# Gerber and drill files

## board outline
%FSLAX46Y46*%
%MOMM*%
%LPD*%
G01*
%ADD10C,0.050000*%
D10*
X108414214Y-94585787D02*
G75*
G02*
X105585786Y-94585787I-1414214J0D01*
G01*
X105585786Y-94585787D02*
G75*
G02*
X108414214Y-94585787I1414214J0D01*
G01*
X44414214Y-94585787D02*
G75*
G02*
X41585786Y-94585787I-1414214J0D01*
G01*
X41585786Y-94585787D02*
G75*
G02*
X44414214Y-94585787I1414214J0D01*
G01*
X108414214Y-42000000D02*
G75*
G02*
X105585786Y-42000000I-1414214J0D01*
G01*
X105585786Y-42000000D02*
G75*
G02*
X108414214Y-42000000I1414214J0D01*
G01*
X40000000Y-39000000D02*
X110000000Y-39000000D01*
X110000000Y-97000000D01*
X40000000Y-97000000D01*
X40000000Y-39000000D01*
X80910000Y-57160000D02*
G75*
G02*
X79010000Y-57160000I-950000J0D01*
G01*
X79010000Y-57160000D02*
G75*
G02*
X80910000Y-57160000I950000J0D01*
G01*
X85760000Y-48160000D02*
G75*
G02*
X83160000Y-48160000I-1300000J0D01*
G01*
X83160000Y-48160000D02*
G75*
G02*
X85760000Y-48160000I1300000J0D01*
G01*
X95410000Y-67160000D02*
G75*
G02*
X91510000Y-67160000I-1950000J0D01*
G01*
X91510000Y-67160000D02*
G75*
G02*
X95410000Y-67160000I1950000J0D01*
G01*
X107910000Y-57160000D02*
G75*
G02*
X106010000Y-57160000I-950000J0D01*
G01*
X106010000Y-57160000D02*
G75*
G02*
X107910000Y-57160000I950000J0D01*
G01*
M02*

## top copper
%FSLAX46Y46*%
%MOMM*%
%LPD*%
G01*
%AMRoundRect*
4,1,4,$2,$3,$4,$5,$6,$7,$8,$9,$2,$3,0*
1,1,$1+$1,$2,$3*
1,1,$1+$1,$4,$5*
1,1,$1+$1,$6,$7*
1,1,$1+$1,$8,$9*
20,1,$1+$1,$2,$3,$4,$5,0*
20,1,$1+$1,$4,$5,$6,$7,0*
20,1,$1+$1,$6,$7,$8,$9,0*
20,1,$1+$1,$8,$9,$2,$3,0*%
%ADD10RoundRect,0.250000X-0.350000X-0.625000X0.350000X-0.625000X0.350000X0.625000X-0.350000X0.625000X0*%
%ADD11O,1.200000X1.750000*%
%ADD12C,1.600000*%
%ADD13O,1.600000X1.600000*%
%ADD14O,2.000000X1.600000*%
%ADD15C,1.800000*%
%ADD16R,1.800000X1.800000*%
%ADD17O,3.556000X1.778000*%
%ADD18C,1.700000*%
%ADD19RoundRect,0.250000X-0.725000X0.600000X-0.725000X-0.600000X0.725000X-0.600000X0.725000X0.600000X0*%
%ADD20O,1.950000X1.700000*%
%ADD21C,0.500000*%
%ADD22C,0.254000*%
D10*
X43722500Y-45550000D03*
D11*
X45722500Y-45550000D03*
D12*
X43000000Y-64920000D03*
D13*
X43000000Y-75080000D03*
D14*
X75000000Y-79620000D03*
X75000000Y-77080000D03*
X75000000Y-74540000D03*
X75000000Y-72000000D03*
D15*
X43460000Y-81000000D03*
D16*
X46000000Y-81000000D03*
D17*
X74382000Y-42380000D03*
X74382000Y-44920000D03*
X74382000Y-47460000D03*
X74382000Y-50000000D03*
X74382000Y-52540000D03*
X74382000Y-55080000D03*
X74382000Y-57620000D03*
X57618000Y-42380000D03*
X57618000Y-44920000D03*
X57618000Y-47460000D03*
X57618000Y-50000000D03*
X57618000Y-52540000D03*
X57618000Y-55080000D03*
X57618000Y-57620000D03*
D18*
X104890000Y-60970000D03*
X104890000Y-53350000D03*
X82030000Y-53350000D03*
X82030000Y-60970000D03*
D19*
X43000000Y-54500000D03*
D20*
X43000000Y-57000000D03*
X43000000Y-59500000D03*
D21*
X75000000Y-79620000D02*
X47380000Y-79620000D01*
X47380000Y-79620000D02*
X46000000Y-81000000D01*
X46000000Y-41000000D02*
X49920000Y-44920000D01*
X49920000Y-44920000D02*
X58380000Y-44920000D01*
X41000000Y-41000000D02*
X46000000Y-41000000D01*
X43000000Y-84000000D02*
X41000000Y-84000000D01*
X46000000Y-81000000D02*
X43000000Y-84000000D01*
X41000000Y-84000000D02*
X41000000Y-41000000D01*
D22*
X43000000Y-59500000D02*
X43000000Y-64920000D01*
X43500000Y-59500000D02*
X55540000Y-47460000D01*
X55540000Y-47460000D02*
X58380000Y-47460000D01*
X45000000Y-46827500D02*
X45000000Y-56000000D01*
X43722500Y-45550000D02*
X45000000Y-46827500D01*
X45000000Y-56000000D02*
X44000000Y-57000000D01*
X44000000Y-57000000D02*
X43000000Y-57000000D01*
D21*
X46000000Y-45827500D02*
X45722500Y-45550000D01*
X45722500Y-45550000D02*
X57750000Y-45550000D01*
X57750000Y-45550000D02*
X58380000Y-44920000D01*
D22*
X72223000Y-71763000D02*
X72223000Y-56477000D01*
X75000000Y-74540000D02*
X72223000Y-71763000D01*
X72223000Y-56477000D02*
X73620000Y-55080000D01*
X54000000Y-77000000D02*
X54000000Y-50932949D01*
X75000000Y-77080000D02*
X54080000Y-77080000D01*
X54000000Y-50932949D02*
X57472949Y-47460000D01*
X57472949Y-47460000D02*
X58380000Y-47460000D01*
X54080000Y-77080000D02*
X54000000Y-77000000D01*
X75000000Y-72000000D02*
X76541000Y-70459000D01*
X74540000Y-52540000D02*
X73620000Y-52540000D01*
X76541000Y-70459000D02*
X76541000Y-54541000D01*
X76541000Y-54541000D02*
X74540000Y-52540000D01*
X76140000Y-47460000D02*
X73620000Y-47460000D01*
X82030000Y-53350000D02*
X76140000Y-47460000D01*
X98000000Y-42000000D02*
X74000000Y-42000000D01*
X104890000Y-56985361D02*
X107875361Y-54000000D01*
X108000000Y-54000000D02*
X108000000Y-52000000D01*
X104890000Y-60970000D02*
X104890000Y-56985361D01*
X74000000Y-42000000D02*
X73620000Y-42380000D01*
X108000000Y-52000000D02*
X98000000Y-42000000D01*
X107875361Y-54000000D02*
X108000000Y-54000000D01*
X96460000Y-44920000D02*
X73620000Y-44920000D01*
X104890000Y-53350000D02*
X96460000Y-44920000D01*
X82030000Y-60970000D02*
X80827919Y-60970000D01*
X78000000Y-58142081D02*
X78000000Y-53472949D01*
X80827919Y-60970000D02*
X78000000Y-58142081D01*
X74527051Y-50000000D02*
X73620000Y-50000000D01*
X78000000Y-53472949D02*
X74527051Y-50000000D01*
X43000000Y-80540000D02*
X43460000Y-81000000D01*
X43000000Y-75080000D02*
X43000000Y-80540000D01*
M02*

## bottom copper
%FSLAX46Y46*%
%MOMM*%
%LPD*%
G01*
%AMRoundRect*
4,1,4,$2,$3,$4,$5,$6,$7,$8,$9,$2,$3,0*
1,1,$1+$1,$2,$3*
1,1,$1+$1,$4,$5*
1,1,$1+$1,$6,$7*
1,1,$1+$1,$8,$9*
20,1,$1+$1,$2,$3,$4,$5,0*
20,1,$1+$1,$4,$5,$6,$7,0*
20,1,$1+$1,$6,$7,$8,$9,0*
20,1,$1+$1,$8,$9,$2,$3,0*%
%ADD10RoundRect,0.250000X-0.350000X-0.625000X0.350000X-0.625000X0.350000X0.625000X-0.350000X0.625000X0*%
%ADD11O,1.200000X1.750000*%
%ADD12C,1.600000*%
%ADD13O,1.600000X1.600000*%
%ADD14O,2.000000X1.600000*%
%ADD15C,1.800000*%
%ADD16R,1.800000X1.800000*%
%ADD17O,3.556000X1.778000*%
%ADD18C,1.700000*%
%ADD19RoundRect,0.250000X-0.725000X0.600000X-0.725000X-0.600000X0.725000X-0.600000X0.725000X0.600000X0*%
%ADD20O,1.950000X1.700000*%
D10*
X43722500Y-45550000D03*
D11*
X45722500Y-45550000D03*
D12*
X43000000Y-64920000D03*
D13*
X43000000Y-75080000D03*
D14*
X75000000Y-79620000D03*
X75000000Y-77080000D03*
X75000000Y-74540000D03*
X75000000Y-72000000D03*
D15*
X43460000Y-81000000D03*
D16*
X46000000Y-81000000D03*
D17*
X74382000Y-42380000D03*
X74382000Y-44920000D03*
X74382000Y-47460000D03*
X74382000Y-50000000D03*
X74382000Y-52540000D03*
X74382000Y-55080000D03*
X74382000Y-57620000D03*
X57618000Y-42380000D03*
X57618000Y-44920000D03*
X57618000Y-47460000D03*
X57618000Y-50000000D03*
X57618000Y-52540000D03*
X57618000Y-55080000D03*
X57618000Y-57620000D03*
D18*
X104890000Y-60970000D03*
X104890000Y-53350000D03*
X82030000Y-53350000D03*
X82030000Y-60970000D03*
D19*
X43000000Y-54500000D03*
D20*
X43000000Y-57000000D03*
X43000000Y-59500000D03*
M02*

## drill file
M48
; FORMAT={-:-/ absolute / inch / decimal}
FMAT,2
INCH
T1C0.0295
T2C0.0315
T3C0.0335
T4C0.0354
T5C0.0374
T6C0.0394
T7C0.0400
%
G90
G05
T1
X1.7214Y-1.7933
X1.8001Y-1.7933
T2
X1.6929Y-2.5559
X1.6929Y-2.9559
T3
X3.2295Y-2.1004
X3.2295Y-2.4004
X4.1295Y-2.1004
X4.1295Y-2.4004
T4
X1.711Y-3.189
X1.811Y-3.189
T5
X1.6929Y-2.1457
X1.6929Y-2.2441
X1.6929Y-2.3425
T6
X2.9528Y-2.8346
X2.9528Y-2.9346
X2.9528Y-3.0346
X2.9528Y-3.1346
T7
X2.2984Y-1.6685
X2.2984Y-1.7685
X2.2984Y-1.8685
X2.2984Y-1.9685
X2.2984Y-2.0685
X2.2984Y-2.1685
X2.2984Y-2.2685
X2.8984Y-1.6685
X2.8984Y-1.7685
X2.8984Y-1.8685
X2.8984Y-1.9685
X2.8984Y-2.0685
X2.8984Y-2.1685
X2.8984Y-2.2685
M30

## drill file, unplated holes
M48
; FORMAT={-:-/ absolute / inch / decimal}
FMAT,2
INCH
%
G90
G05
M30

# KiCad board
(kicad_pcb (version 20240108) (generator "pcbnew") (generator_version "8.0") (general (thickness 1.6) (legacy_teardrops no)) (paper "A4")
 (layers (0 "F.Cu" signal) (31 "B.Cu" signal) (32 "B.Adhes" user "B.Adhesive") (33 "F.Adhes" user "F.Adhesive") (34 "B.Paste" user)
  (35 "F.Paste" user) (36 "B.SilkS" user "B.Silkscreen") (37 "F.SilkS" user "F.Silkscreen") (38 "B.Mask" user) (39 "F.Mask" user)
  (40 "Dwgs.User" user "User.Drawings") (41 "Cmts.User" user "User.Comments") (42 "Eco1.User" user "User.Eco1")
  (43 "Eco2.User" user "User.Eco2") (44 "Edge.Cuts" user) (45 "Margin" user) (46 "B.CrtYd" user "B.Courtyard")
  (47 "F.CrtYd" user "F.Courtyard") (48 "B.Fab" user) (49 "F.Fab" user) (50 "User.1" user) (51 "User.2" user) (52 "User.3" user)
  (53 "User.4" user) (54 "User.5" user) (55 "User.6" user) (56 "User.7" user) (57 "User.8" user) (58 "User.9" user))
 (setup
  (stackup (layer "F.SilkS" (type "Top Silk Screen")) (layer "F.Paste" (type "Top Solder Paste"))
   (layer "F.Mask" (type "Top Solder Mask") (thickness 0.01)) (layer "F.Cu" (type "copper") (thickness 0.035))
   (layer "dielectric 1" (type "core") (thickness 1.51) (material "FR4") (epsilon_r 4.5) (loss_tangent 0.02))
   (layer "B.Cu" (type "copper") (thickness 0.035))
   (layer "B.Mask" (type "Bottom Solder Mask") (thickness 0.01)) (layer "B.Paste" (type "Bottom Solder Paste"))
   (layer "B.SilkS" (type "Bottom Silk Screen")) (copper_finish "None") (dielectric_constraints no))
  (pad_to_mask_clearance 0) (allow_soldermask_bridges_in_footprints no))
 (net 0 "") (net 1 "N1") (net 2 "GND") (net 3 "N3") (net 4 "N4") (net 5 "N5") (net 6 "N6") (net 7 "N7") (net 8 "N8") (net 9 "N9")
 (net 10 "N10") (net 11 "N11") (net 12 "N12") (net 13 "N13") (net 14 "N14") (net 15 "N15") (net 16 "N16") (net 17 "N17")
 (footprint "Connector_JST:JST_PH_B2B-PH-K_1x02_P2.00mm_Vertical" (layer "B.Cu") (at 43.7225 45.55)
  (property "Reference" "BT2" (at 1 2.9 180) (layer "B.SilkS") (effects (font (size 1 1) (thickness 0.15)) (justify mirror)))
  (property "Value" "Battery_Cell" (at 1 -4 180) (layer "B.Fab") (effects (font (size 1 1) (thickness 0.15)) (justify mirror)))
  (pad "1" thru_hole roundrect (at 0 0) (size 1.2 1.75) (drill 0.75) (layers "*.Cu" "*.Mask") (remove_unused_layers no)
   (roundrect_rratio 0.208333) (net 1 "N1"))
  (pad "2" thru_hole oval (at 2 0) (size 1.2 1.75) (drill 0.75) (layers "*.Cu" "*.Mask") (remove_unused_layers no) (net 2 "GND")))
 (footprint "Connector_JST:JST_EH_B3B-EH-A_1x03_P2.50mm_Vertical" (layer "B.Cu") (at 43 54.5 -90)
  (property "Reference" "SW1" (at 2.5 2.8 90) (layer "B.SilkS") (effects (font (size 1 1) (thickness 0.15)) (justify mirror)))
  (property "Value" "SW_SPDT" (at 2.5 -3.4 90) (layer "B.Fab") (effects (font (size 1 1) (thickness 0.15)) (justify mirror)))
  (pad "1" thru_hole roundrect (at 0 0 270) (size 1.7 1.95) (drill 0.95) (layers "*.Cu" "*.Mask") (remove_unused_layers no)
   (roundrect_rratio 0.147059) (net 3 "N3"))
  (pad "2" thru_hole oval (at 2.5 0 270) (size 1.7 1.95) (drill 0.95) (layers "*.Cu" "*.Mask") (remove_unused_layers no) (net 1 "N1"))
  (pad "3" thru_hole oval (at 5 0 270) (size 1.7 1.95) (drill 0.95) (layers "*.Cu" "*.Mask") (remove_unused_layers no) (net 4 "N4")))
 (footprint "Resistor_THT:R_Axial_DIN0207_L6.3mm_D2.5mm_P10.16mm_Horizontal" (layer "B.Cu") (at 43 64.92 -90)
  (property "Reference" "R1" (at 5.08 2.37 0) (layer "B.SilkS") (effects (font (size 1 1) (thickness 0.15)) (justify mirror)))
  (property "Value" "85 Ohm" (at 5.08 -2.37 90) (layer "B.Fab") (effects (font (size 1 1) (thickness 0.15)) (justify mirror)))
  (pad "1" thru_hole circle (at 0 0 270) (size 1.6 1.6) (drill 0.8) (layers "*.Cu" "*.Mask") (remove_unused_layers no) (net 4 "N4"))
  (pad "2" thru_hole oval (at 10.16 0 270) (size 1.6 1.6) (drill 0.8) (layers "*.Cu" "*.Mask") (remove_unused_layers no) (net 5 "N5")))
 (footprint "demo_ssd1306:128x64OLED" (layer "B.Cu") (at 64.4 76 90)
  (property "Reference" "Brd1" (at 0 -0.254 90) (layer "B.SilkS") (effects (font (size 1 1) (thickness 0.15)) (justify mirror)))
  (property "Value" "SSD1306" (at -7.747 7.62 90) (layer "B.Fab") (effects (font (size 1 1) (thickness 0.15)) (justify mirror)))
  (pad "1" thru_hole oval (at -3.62 10.6) (size 2 1.6) (drill 1) (layers "*.Cu" "*.Mask") (remove_unused_layers no) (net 2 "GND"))
  (pad "2" thru_hole oval (at -1.08 10.6) (size 2 1.6) (drill 1) (layers "*.Cu" "*.Mask") (remove_unused_layers no) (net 4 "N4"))
  (pad "3" thru_hole oval (at 1.46 10.6) (size 2 1.6) (drill 1) (layers "*.Cu" "*.Mask") (remove_unused_layers no) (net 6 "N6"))
  (pad "4" thru_hole oval (at 4 10.6) (size 2 1.6) (drill 1) (layers "*.Cu" "*.Mask") (remove_unused_layers no) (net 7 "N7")))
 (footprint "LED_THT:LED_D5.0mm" (layer "B.Cu") (at 46 81 180)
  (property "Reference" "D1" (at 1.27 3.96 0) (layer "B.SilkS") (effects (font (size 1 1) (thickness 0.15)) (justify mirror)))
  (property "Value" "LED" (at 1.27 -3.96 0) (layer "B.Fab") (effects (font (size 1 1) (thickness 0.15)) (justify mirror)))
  (pad "1" thru_hole rect (at 0 0 180) (size 1.8 1.8) (drill 0.9) (layers "*.Cu" "*.Mask") (remove_unused_layers no) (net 2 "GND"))
  (pad "2" thru_hole circle (at 2.54 0 180) (size 1.8 1.8) (drill 0.9) (layers "*.Cu" "*.Mask") (remove_unused_layers no) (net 5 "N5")))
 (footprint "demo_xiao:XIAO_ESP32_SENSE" (layer "B.Cu") (at 66 50 180)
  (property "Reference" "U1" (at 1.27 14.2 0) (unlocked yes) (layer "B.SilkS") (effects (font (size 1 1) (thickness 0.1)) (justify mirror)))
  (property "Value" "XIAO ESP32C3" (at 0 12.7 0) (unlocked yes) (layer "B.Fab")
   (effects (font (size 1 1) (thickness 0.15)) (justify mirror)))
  (pad "1" thru_hole oval (at -7.62 7.62 180) (size 3.556 1.778) (drill 1.016 (offset -0.762 0)) (layers "*.Cu" "*.Mask")
   (remove_unused_layers no) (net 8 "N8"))
  (pad "2" thru_hole oval (at -7.62 5.08 180) (size 3.556 1.778) (drill 1.016 (offset -0.762 0)) (layers "*.Cu" "*.Mask")
   (remove_unused_layers no) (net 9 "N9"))
  (pad "3" thru_hole oval (at -7.62 2.54 180) (size 3.556 1.778) (drill 1.016 (offset -0.762 0)) (layers "*.Cu" "*.Mask")
   (remove_unused_layers no) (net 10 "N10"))
  (pad "4" thru_hole oval (at -7.62 0 180) (size 3.556 1.778) (drill 1.016 (offset -0.762 0)) (layers "*.Cu" "*.Mask")
   (remove_unused_layers no) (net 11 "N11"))
  (pad "5" thru_hole oval (at -7.62 -2.54 180) (size 3.556 1.778) (drill 1.016 (offset -0.762 0)) (layers "*.Cu" "*.Mask")
   (remove_unused_layers no) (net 7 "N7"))
  (pad "6" thru_hole oval (at -7.62 -5.08 180) (size 3.556 1.778) (drill 1.016 (offset -0.762 0)) (layers "*.Cu" "*.Mask")
   (remove_unused_layers no) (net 6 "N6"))
  (pad "7" thru_hole oval (at -7.62 -7.62 180) (size 3.556 1.778) (drill 1.016 (offset -0.762 0)) (layers "*.Cu" "*.Mask")
   (remove_unused_layers no) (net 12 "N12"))
  (pad "8" thru_hole oval (at 7.62 7.62 180) (size 3.556 1.778) (drill 1.016 (offset 0.762 0)) (layers "*.Cu" "*.Mask")
   (remove_unused_layers no) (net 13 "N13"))
  (pad "9" thru_hole oval (at 7.62 5.08 180) (size 3.556 1.778) (drill 1.016 (offset 0.762 0)) (layers "*.Cu" "*.Mask")
   (remove_unused_layers no) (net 2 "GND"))
  (pad "10" thru_hole oval (at 7.62 2.54 180) (size 3.556 1.778) (drill 1.016 (offset 0.762 0)) (layers "*.Cu" "*.Mask")
   (remove_unused_layers no) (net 4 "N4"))
  (pad "11" thru_hole oval (at 7.62 0 180) (size 3.556 1.778) (drill 1.016 (offset 0.762 0)) (layers "*.Cu" "*.Mask")
   (remove_unused_layers no) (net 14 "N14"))
  (pad "12" thru_hole oval (at 7.62 -2.54 180) (size 3.556 1.778) (drill 1.016 (offset 0.762 0)) (layers "*.Cu" "*.Mask")
   (remove_unused_layers no) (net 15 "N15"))
  (pad "13" thru_hole oval (at 7.62 -5.08 180) (size 3.556 1.778) (drill 1.016 (offset 0.762 0)) (layers "*.Cu" "*.Mask")
   (remove_unused_layers no) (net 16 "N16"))
  (pad "14" thru_hole oval (at 7.62 -7.62 180) (size 3.556 1.778) (drill 1.016 (offset 0.762 0)) (layers "*.Cu" "*.Mask")
   (remove_unused_layers no) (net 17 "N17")))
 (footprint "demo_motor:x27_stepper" (layer "B.Cu") (at 96 47)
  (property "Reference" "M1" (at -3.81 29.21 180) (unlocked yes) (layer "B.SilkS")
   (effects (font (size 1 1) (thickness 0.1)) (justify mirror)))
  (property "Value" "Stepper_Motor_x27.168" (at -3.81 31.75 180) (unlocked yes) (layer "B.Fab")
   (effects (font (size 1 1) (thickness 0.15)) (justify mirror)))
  (fp_circle (center -16.04 10.16) (end -15.09 10.16) (stroke (width 0.05) (type default)) (fill none) (layer "Edge.Cuts"))
  (fp_circle (center -11.54 1.16) (end -10.24 1.16) (stroke (width 0.05) (type default)) (fill none) (layer "Edge.Cuts"))
  (fp_circle (center -2.54 20.16) (end -0.59 20.16) (stroke (width 0.05) (type default)) (fill none) (layer "Edge.Cuts"))
  (fp_circle (center 10.96 10.16) (end 11.91 10.16) (stroke (width 0.05) (type default)) (fill none) (layer "Edge.Cuts"))
  (pad "1" thru_hole circle (at 8.89 13.97) (size 1.7 1.7) (drill 0.85) (layers "*.Cu" "*.Mask") (remove_unused_layers no) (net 8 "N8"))
  (pad "2" thru_hole circle (at 8.89 6.35) (size 1.7 1.7) (drill 0.85) (layers "*.Cu" "*.Mask") (remove_unused_layers no) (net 9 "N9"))
  (pad "3" thru_hole circle (at -13.97 6.35) (size 1.7 1.7) (drill 0.85) (layers "*.Cu" "*.Mask") (remove_unused_layers no) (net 10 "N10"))
  (pad "4" thru_hole circle (at -13.97 13.97) (size 1.7 1.7) (drill 0.85) (layers "*.Cu" "*.Mask") (remove_unused_layers no) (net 11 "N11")))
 (gr_rect (start 40 39) (end 110 97) (stroke (width 0.05) (type default)) (fill none) (layer "Edge.Cuts"))
 (gr_circle (center 43 94.585787) (end 44 95.585787) (stroke (width 0.05) (type default)) (fill none) (layer "Edge.Cuts"))
 (gr_circle (center 107 94.585787) (end 108 95.585787) (stroke (width 0.05) (type default)) (fill none) (layer "Edge.Cuts"))
 (gr_circle (center 107 42) (end 108 43) (stroke (width 0.05) (type default)) (fill none) (layer "Edge.Cuts"))
 (segment (start 72.223 71.763) (end 72.223 56.477) (width 0.254) (layer "F.Cu") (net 6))
 (segment (start 75 74.54) (end 72.223 71.763) (width 0.254) (layer "F.Cu") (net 6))
 (segment (start 72.223 56.477) (end 73.62 55.08) (width 0.254) (layer "F.Cu") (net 6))
 (segment (start 54 77) (end 54 50.932949) (width 0.254) (layer "F.Cu") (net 4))
 (segment (start 75 77.08) (end 54.08 77.08) (width 0.254) (layer "F.Cu") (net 4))
 (segment (start 43.5 59.5) (end 55.54 47.46) (width 0.254) (layer "F.Cu") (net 4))
 (segment (start 54 50.932949) (end 57.472949 47.46) (width 0.254) (layer "F.Cu") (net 4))
 (segment (start 57.472949 47.46) (end 58.38 47.46) (width 0.254) (layer "F.Cu") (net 4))
 (segment (start 54.08 77.08) (end 54 77) (width 0.254) (layer "F.Cu") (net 4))
 (segment (start 55.54 47.46) (end 58.38 47.46) (width 0.254) (layer "F.Cu") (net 4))
 (segment (start 43 59.5) (end 43 64.92) (width 0.254) (layer "F.Cu") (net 4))
 (segment (start 43 84) (end 41 84) (width 0.5) (layer "F.Cu") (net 2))
 (segment (start 46 41) (end 49.92 44.92) (width 0.5) (layer "F.Cu") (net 2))
 (segment (start 46 81) (end 43 84) (width 0.5) (layer "F.Cu") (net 2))
 (segment (start 75 79.62) (end 47.38 79.62) (width 0.5) (layer "F.Cu") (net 2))
 (segment (start 49.92 44.92) (end 58.38 44.92) (width 0.5) (layer "F.Cu") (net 2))
 (segment (start 46 45.8275) (end 45.7225 45.55) (width 0.5) (layer "F.Cu") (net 2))
 (segment (start 41 41) (end 46 41) (width 0.5) (layer "F.Cu") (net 2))
 (segment (start 47.38 79.62) (end 46 81) (width 0.5) (layer "F.Cu") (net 2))
 (segment (start 45.7225 45.55) (end 57.75 45.55) (width 0.5) (layer "F.Cu") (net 2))
 (segment (start 57.75 45.55) (end 58.38 44.92) (width 0.5) (layer "F.Cu") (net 2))
 (segment (start 41 84) (end 41 41) (width 0.5) (layer "F.Cu") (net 2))
 (segment (start 75 72) (end 76.541 70.459) (width 0.254) (layer "F.Cu") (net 7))
 (segment (start 74.54 52.54) (end 73.62 52.54) (width 0.254) (layer "F.Cu") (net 7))
 (segment (start 76.541 70.459) (end 76.541 54.541) (width 0.254) (layer "F.Cu") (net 7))
 (segment (start 76.541 54.541) (end 74.54 52.54) (width 0.254) (layer "F.Cu") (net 7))
 (segment (start 44 57) (end 43 57) (width 0.254) (layer "F.Cu") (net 1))
 (segment (start 45 46.8275) (end 45 56) (width 0.254) (layer "F.Cu") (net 1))
 (segment (start 43.7225 45.55) (end 45 46.8275) (width 0.254) (layer "F.Cu") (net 1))
 (segment (start 45 56) (end 44 57) (width 0.254) (layer "F.Cu") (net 1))
 (segment (start 43 75.08) (end 43 80.54) (width 0.254) (layer "F.Cu") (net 5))
 (segment (start 43 80.54) (end 43.46 81) (width 0.254) (layer "F.Cu") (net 5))
 (segment (start 76.14 47.46) (end 73.62 47.46) (width 0.254) (layer "F.Cu") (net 10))
 (segment (start 82.03 53.35) (end 76.14 47.46) (width 0.254) (layer "F.Cu") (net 10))
 (segment (start 98 42) (end 74 42) (width 0.254) (layer "F.Cu") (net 8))
 (segment (start 104.89 56.985361) (end 107.875361 54) (width 0.254) (layer "F.Cu") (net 8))
 (segment (start 108 54) (end 108 52) (width 0.254) (layer "F.Cu") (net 8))
 (segment (start 104.89 60.97) (end 104.89 56.985361) (width 0.254) (layer "F.Cu") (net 8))
 (segment (start 74 42) (end 73.62 42.38) (width 0.254) (layer "F.Cu") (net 8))
 (segment (start 108 52) (end 98 42) (width 0.254) (layer "F.Cu") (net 8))
 (segment (start 107.875361 54) (end 108 54) (width 0.254) (layer "F.Cu") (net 8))
 (segment (start 96.46 44.92) (end 73.62 44.92) (width 0.254) (layer "F.Cu") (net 9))
 (segment (start 104.89 53.35) (end 96.46 44.92) (width 0.254) (layer "F.Cu") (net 9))
 (segment (start 82.03 60.97) (end 80.827919 60.97) (width 0.254) (layer "F.Cu") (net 11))
 (segment (start 78 58.142081) (end 78 53.472949) (width 0.254) (layer "F.Cu") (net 11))
 (segment (start 80.827919 60.97) (end 78 58.142081) (width 0.254) (layer "F.Cu") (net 11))
 (segment (start 74.527051 50) (end 73.62 50) (width 0.254) (layer "F.Cu") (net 11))
 (segment (start 78 53.472949) (end 74.527051 50) (width 0.254) (layer "F.Cu") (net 11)))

